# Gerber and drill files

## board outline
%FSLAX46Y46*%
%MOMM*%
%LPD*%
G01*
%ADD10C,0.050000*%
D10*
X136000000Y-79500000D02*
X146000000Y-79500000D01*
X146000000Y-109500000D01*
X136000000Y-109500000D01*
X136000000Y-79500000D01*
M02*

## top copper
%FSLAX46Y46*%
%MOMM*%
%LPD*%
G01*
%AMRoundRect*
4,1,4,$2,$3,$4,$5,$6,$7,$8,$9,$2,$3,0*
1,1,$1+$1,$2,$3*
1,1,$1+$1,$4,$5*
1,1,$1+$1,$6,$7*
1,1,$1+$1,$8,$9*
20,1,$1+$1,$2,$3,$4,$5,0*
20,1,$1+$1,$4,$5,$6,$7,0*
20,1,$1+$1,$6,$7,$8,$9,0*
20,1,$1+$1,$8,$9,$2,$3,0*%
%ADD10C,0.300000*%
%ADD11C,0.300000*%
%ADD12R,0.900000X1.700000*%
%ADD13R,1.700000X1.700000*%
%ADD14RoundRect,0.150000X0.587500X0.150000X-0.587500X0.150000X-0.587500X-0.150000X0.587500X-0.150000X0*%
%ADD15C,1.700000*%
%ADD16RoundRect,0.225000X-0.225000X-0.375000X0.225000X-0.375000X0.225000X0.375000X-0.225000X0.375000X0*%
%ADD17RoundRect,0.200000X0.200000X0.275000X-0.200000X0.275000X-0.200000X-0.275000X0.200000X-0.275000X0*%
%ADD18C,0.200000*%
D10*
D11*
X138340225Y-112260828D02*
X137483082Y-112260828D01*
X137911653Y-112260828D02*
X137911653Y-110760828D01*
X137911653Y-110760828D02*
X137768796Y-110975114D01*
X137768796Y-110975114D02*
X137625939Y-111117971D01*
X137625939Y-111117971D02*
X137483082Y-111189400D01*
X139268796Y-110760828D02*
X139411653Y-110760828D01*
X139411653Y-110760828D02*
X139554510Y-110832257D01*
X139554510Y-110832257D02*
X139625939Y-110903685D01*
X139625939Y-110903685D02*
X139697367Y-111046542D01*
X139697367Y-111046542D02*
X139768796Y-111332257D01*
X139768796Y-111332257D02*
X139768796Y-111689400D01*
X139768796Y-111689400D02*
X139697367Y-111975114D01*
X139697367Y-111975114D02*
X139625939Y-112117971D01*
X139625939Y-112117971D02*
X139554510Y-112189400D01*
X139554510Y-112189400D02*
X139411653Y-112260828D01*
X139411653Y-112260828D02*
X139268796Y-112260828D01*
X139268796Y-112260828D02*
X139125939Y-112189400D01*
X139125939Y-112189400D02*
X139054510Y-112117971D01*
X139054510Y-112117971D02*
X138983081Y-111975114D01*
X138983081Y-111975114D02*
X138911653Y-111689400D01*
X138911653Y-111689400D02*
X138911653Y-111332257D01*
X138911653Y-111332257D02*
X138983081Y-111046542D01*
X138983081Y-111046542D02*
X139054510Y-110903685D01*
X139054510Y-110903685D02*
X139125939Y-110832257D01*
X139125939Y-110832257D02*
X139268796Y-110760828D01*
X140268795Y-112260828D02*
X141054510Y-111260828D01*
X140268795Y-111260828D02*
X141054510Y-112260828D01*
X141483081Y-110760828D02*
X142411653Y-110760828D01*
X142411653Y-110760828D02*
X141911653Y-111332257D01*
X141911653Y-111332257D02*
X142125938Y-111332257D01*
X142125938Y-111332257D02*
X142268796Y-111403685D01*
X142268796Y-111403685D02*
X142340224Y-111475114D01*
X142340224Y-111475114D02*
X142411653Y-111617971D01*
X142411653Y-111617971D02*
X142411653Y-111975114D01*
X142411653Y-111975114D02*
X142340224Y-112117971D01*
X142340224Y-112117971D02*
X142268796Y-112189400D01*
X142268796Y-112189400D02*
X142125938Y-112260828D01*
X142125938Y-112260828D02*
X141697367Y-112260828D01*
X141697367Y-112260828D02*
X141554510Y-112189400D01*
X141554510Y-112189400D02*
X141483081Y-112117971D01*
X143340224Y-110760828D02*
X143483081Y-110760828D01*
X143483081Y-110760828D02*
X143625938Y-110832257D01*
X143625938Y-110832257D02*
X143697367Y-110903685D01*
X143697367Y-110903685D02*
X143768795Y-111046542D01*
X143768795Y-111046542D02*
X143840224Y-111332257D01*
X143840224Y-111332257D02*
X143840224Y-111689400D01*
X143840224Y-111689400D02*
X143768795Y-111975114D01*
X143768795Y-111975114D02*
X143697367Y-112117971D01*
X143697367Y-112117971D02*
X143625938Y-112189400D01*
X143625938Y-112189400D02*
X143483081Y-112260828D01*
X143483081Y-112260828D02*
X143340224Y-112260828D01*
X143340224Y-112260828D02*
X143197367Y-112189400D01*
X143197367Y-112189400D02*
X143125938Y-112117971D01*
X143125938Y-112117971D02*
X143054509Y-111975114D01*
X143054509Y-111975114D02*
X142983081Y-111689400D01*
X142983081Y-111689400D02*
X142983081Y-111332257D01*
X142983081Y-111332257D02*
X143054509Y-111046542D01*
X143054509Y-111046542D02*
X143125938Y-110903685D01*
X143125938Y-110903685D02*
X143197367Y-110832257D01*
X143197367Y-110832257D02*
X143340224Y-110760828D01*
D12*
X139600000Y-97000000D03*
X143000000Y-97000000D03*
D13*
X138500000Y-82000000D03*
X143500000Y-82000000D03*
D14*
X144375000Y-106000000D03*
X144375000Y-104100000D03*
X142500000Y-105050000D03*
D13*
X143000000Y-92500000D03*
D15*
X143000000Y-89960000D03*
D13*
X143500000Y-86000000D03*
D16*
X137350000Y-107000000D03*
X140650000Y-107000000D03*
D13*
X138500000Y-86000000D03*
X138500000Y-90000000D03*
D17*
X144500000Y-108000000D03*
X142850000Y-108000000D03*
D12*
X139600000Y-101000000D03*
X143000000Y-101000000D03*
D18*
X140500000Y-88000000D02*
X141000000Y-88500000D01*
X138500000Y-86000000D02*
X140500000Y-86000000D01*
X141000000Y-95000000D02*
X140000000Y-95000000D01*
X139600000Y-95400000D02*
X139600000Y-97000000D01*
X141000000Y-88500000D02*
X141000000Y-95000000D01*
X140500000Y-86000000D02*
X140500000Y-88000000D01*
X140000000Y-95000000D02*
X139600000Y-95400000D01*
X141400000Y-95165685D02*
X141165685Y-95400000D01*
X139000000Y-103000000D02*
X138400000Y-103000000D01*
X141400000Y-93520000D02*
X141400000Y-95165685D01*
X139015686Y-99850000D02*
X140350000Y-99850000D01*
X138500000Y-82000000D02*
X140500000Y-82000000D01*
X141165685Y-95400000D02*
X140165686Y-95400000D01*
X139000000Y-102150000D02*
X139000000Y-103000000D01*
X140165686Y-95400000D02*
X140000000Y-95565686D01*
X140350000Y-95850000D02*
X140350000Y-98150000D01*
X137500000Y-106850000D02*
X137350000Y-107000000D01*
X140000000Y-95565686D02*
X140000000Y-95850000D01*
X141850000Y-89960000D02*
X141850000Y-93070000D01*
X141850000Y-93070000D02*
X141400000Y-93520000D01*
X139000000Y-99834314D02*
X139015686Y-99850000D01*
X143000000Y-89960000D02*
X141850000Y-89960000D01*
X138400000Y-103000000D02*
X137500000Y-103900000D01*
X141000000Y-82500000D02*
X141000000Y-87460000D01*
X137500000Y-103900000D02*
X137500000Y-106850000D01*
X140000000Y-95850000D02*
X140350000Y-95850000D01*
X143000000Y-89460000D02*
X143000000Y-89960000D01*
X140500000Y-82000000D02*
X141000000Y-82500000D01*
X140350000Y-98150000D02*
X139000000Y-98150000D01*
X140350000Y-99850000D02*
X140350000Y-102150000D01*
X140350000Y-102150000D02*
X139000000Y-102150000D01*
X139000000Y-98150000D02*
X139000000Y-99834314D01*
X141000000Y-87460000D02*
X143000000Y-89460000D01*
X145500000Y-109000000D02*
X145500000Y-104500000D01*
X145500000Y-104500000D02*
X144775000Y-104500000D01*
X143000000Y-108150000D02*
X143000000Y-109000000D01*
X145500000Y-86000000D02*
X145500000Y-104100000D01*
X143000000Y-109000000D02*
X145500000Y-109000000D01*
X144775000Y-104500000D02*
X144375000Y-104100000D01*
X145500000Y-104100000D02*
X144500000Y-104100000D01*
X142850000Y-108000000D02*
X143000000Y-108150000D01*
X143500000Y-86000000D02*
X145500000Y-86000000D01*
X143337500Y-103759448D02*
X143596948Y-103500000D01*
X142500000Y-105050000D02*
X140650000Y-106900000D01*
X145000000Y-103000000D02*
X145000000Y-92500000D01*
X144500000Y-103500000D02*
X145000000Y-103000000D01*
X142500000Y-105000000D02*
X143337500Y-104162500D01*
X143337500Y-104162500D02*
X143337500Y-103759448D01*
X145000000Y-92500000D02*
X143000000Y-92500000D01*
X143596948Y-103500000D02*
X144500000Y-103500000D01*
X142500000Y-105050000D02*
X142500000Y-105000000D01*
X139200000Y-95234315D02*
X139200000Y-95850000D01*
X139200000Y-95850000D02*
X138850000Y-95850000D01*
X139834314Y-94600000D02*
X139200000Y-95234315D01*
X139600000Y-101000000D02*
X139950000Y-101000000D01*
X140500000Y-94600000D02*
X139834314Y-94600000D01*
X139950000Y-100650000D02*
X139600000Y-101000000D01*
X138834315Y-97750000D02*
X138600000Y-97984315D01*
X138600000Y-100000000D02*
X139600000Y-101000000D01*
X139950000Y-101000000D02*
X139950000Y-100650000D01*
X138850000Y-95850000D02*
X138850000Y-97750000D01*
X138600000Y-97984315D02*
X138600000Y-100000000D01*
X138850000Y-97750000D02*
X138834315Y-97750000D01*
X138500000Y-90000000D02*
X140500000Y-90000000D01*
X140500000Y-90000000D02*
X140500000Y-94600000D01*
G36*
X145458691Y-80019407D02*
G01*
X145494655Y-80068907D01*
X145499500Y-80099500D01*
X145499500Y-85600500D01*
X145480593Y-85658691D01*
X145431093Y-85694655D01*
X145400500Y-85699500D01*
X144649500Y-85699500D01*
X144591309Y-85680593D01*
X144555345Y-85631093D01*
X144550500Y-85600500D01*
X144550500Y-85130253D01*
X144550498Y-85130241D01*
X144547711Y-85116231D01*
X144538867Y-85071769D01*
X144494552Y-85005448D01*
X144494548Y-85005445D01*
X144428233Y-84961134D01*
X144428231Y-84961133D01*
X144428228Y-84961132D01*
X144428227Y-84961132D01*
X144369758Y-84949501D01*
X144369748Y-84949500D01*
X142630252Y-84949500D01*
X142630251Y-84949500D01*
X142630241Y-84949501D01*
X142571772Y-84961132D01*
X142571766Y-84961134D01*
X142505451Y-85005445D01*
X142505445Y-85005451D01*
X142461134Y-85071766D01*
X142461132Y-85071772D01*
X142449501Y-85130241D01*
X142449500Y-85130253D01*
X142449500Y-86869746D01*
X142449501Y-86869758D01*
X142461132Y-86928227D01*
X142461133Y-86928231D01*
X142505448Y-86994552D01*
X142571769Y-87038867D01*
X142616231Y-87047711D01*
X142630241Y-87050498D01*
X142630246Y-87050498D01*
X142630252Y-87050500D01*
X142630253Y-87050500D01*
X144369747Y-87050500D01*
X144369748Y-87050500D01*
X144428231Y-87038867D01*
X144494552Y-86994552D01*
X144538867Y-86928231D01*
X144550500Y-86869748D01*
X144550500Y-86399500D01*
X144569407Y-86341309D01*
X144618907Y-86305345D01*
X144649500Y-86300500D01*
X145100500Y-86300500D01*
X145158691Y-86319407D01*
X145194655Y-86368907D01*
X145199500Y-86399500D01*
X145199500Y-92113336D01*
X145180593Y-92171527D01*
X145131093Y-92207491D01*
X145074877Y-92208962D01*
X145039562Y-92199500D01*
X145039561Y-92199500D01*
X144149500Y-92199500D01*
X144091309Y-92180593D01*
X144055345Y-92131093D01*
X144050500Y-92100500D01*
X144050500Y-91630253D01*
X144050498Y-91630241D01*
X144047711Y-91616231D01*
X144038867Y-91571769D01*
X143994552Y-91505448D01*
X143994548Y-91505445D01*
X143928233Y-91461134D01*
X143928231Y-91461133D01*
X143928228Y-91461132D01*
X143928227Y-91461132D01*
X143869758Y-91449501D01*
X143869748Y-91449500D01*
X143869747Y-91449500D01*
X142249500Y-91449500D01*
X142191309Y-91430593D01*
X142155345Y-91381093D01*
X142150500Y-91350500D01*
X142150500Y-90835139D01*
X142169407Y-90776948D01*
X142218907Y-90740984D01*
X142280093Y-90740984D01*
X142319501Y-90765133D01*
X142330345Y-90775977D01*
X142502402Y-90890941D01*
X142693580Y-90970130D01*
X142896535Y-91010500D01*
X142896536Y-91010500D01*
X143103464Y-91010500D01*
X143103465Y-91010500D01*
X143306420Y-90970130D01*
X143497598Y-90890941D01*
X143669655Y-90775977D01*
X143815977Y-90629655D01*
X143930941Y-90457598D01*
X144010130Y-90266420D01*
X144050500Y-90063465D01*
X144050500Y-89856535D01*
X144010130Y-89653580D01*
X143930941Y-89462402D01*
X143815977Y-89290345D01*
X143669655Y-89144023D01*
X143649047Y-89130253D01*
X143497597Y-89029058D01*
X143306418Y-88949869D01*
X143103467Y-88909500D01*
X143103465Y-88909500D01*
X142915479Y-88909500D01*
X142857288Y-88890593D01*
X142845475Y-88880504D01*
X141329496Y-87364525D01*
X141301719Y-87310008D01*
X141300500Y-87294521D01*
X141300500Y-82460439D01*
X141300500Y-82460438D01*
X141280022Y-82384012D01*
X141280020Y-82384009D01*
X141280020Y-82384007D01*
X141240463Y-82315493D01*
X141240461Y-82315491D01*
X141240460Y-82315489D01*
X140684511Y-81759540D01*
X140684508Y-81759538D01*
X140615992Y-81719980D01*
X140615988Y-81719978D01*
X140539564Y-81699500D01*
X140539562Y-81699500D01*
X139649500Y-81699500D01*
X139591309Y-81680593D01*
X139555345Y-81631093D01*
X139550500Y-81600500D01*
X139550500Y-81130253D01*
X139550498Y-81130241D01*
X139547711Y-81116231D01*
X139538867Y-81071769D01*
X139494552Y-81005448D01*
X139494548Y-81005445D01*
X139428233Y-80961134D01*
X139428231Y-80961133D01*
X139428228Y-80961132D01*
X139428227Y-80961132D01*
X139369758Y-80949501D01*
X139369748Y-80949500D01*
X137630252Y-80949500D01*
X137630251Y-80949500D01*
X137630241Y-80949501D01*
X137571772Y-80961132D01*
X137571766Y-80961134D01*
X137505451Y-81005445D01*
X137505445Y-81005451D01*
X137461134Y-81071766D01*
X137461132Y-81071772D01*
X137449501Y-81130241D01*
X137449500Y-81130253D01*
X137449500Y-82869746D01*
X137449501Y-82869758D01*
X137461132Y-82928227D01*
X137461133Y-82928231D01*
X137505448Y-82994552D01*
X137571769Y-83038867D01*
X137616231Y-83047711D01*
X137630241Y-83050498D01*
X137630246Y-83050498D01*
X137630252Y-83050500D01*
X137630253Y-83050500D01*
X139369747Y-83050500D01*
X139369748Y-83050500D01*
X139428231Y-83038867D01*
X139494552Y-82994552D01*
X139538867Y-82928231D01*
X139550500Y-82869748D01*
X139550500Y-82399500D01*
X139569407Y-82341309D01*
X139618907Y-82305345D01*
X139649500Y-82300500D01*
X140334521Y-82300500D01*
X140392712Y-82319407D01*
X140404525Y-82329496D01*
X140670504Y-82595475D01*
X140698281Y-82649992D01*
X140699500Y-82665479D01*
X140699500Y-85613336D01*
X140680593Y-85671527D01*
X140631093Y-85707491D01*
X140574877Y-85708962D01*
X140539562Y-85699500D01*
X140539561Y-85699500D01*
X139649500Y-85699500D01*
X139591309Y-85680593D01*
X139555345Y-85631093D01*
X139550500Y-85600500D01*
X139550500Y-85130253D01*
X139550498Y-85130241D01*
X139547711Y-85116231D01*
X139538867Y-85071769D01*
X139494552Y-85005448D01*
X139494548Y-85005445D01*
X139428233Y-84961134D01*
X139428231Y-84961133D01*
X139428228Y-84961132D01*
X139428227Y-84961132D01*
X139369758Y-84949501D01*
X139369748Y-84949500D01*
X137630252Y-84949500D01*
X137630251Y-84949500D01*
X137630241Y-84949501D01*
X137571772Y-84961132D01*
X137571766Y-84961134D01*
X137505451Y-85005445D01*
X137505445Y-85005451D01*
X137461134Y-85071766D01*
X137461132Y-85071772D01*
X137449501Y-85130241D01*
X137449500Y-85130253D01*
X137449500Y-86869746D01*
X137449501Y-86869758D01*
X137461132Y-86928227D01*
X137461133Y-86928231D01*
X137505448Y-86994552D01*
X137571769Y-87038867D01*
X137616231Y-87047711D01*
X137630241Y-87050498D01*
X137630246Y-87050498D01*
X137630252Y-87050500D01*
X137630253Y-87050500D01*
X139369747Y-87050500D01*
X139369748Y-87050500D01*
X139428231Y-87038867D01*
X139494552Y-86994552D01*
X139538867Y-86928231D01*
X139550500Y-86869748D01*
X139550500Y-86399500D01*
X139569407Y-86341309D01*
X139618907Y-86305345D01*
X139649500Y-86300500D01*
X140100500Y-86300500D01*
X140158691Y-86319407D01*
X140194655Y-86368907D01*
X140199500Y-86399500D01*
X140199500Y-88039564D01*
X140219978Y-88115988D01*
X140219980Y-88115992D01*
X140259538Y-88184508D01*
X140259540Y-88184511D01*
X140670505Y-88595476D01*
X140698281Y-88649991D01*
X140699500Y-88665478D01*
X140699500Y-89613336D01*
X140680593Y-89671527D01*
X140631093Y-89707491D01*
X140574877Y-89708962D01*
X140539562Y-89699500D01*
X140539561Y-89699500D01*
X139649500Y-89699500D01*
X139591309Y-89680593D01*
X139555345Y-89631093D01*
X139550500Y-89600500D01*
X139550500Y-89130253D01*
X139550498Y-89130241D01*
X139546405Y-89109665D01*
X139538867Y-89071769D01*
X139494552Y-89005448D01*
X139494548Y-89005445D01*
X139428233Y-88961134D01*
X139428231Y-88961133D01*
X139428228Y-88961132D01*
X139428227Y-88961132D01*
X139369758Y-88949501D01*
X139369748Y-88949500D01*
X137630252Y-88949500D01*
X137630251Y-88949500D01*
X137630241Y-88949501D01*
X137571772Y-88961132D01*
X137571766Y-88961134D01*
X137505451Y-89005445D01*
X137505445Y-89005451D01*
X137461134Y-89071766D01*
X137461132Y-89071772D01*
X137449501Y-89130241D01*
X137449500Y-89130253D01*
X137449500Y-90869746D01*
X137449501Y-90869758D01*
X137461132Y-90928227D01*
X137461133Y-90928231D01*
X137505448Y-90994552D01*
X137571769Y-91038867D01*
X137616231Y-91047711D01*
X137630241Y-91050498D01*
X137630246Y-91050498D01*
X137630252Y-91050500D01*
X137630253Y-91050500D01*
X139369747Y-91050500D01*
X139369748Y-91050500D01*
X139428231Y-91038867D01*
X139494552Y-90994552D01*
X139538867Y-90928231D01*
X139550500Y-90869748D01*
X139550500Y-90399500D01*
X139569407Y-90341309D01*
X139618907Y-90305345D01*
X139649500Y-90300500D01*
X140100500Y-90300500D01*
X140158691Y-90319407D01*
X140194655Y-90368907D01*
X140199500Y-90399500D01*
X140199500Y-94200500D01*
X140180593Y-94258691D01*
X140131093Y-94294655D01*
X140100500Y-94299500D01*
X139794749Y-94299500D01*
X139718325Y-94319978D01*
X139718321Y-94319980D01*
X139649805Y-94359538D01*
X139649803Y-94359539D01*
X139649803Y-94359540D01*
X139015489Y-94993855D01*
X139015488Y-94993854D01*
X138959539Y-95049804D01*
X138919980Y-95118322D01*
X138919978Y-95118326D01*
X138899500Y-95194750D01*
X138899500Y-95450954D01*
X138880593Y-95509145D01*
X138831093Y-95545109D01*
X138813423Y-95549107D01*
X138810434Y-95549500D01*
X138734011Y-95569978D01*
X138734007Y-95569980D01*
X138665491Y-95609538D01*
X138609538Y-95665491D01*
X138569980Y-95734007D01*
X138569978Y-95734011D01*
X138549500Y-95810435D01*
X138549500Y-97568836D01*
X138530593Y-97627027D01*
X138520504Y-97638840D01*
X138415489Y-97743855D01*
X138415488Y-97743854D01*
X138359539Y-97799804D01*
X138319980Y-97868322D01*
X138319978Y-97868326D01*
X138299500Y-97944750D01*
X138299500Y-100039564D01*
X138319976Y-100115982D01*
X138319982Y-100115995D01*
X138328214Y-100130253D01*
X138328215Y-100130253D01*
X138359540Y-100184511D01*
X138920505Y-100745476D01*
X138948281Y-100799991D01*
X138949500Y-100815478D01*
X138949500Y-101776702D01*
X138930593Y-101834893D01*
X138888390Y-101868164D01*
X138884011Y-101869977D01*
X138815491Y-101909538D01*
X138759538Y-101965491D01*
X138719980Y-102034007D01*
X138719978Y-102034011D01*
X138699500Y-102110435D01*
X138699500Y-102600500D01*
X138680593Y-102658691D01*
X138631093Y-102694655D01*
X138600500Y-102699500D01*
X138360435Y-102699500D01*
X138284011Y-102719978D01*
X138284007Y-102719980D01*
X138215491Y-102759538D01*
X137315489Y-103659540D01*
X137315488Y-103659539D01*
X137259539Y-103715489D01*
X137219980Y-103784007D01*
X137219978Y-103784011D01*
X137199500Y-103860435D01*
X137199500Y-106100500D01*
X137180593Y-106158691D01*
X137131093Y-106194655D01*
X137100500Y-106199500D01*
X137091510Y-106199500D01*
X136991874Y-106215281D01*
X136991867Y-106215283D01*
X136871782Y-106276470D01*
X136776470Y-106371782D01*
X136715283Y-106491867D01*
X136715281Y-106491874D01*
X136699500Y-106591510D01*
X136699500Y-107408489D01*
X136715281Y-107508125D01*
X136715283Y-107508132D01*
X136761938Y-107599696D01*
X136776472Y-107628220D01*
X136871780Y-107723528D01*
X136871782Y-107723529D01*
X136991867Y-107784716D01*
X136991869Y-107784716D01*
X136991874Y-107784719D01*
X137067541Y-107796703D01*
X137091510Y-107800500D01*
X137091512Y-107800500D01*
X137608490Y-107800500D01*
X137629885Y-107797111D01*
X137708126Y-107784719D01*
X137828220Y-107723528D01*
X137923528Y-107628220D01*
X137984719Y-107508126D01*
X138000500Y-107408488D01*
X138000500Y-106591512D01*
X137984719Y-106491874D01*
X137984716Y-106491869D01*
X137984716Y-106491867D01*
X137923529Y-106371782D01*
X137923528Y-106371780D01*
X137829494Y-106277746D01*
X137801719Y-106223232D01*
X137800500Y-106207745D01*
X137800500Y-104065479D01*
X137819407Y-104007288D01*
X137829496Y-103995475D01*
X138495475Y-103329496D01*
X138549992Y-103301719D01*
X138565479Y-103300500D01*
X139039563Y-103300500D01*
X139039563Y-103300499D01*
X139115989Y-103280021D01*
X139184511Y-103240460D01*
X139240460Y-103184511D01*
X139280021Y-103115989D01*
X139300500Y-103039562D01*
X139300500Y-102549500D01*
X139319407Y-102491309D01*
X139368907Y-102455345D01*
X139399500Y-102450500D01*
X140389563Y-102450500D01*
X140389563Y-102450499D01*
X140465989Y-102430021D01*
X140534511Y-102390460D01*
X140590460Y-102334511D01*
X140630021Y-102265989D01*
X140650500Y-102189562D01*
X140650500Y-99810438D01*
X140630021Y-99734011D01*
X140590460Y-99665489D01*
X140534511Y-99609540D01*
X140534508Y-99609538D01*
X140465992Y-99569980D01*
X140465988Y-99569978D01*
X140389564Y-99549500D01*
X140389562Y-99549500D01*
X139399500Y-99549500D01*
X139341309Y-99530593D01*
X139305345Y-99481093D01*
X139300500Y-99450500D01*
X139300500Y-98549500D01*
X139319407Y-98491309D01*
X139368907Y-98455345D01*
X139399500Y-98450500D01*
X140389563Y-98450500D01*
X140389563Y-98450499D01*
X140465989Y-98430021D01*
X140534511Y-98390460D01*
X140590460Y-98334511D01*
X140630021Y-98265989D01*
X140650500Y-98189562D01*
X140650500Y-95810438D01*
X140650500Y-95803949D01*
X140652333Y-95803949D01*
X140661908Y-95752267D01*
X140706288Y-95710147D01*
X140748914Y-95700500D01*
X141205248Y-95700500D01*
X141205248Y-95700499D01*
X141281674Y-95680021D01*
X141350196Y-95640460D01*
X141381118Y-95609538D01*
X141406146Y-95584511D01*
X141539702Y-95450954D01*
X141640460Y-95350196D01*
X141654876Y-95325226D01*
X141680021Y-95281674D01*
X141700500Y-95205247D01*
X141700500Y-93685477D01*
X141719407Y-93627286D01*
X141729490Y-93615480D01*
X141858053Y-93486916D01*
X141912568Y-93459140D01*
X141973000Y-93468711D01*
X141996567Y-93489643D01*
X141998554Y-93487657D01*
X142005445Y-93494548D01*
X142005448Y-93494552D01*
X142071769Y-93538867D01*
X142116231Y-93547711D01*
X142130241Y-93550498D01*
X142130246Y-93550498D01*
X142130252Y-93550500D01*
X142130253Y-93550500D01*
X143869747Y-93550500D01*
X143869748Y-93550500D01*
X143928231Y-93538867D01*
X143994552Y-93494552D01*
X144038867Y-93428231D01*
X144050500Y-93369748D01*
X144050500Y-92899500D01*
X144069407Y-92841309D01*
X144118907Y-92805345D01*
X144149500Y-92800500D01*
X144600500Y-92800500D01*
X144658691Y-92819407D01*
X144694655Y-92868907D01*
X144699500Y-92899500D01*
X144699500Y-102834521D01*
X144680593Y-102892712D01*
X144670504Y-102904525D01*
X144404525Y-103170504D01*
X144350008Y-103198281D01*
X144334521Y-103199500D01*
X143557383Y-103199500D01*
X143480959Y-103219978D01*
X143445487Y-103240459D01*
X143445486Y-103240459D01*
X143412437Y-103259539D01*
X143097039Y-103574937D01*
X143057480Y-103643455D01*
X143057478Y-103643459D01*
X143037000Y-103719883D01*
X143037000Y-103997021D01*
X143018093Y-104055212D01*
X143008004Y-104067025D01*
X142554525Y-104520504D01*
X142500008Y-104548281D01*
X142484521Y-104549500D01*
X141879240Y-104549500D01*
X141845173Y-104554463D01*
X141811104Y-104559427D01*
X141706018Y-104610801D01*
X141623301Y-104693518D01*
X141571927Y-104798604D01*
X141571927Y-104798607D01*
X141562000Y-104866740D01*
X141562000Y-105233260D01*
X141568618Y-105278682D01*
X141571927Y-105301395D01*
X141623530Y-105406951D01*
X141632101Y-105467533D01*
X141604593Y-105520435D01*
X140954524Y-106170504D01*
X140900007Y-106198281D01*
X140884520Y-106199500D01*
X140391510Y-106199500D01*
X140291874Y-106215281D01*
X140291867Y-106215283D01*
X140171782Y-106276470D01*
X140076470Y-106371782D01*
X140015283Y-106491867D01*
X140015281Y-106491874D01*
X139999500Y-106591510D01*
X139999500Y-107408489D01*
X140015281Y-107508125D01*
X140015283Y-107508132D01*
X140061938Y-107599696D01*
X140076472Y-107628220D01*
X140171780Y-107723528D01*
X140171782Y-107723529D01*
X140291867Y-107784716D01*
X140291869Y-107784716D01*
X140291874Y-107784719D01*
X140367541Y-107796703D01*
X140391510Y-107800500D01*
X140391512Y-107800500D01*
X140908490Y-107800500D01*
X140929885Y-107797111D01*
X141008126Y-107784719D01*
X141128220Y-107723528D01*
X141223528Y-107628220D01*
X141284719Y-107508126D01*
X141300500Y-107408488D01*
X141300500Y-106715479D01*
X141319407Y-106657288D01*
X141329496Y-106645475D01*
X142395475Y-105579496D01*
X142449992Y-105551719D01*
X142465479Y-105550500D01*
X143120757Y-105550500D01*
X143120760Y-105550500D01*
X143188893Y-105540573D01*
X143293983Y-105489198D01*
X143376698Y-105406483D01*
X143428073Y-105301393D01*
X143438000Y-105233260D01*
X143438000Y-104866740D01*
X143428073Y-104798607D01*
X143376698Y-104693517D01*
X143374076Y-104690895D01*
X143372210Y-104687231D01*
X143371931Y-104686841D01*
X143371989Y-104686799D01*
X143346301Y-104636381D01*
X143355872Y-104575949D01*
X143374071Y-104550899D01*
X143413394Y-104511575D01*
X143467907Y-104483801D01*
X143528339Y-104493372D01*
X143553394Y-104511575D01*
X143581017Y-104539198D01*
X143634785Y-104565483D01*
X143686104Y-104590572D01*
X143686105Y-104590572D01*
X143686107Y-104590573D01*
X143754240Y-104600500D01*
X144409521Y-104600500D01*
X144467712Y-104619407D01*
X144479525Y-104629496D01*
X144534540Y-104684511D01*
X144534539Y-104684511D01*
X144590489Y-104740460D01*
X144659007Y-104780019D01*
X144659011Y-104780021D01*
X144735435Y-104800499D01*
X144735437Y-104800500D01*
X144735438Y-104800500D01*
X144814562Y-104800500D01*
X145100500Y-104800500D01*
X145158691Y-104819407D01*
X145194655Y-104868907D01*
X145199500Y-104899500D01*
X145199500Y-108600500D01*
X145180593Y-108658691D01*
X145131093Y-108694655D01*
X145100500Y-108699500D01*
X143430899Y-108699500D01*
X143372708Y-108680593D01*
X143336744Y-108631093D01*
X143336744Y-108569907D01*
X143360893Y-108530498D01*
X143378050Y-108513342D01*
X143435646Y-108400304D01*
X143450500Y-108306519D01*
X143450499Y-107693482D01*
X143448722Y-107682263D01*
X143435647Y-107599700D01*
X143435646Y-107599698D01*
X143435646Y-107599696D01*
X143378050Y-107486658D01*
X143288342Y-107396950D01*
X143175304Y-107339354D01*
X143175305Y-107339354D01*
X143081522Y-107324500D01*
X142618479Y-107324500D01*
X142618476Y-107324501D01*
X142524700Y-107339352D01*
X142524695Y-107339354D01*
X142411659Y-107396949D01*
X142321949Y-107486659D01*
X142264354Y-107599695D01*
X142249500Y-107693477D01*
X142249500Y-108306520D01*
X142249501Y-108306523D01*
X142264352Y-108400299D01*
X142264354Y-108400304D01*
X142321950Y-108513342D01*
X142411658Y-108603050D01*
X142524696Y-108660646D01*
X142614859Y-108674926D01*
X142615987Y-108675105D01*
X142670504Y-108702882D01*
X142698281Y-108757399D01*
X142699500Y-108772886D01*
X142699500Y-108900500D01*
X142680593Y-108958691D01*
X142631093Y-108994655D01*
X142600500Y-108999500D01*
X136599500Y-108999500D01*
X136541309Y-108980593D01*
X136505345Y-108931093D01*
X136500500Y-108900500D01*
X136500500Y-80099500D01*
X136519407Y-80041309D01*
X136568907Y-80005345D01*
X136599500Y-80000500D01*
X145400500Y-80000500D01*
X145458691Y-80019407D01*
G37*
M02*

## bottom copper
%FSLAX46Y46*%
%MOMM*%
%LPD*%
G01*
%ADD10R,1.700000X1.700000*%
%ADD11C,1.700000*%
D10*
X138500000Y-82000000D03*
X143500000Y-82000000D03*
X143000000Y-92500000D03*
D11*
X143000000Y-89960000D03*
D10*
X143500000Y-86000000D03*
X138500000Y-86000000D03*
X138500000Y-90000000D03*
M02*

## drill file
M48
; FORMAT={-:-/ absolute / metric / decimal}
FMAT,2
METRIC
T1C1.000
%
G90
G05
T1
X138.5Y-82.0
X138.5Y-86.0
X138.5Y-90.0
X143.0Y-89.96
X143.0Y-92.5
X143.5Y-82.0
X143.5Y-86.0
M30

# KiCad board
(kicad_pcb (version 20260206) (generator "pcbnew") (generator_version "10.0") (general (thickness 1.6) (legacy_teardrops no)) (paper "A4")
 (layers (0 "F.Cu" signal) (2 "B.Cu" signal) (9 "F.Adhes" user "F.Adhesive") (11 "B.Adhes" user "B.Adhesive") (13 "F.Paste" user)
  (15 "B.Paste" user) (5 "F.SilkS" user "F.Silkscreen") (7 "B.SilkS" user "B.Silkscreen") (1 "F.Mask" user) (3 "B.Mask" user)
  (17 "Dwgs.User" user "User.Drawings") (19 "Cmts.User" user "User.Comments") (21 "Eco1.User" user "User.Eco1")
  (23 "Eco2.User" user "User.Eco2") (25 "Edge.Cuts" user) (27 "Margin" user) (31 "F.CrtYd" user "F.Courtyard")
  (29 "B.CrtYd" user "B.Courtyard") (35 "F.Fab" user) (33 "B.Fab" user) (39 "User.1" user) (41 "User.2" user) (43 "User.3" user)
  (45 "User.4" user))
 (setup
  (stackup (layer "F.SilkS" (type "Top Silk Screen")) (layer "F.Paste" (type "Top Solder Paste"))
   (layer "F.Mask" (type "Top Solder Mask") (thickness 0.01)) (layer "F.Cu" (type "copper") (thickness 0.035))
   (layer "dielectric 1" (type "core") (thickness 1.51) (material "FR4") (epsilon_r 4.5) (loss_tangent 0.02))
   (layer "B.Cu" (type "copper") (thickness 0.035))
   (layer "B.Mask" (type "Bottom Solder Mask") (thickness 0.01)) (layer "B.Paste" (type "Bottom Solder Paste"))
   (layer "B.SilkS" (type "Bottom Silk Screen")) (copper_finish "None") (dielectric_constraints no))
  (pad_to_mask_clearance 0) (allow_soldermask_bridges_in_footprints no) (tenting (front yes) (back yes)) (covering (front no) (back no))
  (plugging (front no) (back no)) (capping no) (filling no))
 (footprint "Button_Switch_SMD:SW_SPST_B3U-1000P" (layer "F.Cu") (at 141.3 97)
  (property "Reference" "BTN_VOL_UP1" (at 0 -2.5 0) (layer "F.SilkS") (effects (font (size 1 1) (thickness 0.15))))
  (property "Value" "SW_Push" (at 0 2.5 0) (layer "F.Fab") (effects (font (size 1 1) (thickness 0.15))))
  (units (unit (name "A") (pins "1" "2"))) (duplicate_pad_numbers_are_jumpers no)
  (pad "1" smd rect (at -1.7 0) (size 0.9 1.7) (layers "F.Cu" "F.Mask" "F.Paste") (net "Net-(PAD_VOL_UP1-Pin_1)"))
  (pad "2" smd rect (at 1.7 0) (size 0.9 1.7) (layers "F.Cu" "F.Mask" "F.Paste") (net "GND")))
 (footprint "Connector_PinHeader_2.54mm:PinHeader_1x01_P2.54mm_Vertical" (layer "F.Cu") (at 138.5 82)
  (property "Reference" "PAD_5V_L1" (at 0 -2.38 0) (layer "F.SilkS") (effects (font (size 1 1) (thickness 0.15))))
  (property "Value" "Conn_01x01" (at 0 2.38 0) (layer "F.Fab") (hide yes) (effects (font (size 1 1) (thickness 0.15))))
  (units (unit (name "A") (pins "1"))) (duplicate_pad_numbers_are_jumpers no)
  (pad "1" thru_hole rect (at 0 0) (size 1.7 1.7) (drill 1) (layers "*.Cu" "*.Mask") (remove_unused_layers no) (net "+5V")))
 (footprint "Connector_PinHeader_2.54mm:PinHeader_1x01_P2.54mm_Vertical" (layer "F.Cu") (at 143.5 82)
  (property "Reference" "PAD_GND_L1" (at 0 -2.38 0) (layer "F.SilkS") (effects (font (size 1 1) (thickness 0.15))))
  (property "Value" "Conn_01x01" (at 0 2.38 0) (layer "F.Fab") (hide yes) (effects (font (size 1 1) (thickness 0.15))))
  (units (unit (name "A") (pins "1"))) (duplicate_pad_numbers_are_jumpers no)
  (pad "1" thru_hole rect (at 0 0) (size 1.7 1.7) (drill 1) (layers "*.Cu" "*.Mask") (remove_unused_layers no) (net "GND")))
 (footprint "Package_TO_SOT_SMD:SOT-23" (layer "F.Cu") (at 143.4375 105.05 180)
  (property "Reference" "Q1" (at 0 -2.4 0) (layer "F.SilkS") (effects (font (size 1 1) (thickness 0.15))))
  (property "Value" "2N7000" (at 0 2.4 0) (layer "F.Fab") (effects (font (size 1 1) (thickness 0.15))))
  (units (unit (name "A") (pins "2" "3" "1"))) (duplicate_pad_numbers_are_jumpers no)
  (pad "1" smd roundrect (at -0.9375 -0.95 180) (size 1.475 0.6) (layers "F.Cu" "F.Mask" "F.Paste") (roundrect_rratio 0.25) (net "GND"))
  (pad "2" smd roundrect (at -0.9375 0.95 180) (size 1.475 0.6) (layers "F.Cu" "F.Mask" "F.Paste") (roundrect_rratio 0.25)
   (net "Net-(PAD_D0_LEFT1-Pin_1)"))
  (pad "3" smd roundrect (at 0.9375 0 180) (size 1.475 0.6) (layers "F.Cu" "F.Mask" "F.Paste") (roundrect_rratio 0.25) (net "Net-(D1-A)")))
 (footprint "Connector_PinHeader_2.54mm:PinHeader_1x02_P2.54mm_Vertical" (layer "F.Cu") (at 143 92.5 180)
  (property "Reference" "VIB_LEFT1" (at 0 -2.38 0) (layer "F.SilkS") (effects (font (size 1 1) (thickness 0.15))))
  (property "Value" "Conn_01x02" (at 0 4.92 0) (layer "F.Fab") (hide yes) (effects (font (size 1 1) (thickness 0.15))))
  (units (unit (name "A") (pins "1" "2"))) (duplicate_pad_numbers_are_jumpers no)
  (pad "1" thru_hole rect (at 0 0 180) (size 1.7 1.7) (drill 1) (layers "*.Cu" "*.Mask") (remove_unused_layers no) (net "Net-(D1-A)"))
  (pad "2" thru_hole circle (at 0 2.54 180) (size 1.7 1.7) (drill 1) (layers "*.Cu" "*.Mask") (remove_unused_layers no) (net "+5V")))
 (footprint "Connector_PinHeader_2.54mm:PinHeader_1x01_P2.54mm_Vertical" (layer "F.Cu") (at 143.5 86)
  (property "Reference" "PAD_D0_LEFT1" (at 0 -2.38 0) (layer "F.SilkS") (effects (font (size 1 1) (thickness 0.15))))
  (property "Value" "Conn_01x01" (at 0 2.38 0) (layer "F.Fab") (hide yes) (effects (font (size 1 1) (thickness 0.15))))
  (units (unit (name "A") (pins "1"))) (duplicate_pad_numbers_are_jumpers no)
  (pad "1" thru_hole rect (at 0 0) (size 1.7 1.7) (drill 1) (layers "*.Cu" "*.Mask") (remove_unused_layers no)
   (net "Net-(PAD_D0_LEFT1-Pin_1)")))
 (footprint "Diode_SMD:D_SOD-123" (layer "F.Cu") (at 139 107)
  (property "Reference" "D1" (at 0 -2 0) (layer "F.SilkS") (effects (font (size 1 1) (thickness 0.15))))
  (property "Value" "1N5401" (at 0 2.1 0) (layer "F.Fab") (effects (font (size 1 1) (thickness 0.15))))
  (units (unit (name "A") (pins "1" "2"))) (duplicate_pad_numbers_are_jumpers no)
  (pad "1" smd roundrect (at -1.65 0) (size 0.9 1.2) (layers "F.Cu" "F.Mask" "F.Paste") (roundrect_rratio 0.25) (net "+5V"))
  (pad "2" smd roundrect (at 1.65 0) (size 0.9 1.2) (layers "F.Cu" "F.Mask" "F.Paste") (roundrect_rratio 0.25) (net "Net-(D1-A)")))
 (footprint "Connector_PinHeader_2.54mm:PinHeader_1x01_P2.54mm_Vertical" (layer "F.Cu") (at 138.5 86)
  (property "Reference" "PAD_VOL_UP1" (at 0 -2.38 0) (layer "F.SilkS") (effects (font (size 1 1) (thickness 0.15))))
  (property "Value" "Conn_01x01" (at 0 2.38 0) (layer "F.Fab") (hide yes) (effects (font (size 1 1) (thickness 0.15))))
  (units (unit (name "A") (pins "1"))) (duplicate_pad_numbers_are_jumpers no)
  (pad "1" thru_hole rect (at 0 0) (size 1.7 1.7) (drill 1) (layers "*.Cu" "*.Mask") (remove_unused_layers no)
   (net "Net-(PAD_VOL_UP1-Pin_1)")))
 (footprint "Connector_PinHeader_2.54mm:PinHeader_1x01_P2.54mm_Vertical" (layer "F.Cu") (at 138.5 90)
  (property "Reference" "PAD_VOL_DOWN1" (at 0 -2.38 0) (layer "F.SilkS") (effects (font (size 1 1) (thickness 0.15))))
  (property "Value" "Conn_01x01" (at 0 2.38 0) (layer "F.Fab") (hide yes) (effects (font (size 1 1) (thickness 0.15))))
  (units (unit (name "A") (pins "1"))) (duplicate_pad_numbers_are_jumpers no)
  (pad "1" thru_hole rect (at 0 0) (size 1.7 1.7) (drill 1) (layers "*.Cu" "*.Mask") (remove_unused_layers no)
   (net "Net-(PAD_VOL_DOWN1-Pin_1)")))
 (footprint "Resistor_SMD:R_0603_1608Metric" (layer "F.Cu") (at 143.675 108 180)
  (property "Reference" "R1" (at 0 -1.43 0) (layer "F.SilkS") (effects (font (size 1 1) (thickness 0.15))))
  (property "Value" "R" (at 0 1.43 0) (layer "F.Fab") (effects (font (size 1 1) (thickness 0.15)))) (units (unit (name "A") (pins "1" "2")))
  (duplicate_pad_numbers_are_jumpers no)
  (pad "1" smd roundrect (at -0.825 0 180) (size 0.8 0.95) (layers "F.Cu" "F.Mask" "F.Paste") (roundrect_rratio 0.25) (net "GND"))
  (pad "2" smd roundrect (at 0.825 0 180) (size 0.8 0.95) (layers "F.Cu" "F.Mask" "F.Paste") (roundrect_rratio 0.25)
   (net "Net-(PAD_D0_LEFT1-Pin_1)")))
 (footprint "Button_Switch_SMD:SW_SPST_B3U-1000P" (layer "F.Cu") (at 141.3 101)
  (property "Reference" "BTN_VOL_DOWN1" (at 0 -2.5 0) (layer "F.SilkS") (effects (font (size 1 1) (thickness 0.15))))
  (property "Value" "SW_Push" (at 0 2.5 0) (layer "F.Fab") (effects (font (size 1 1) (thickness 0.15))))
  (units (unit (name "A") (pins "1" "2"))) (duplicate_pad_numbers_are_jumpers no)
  (pad "1" smd rect (at -1.7 0) (size 0.9 1.7) (layers "F.Cu" "F.Mask" "F.Paste") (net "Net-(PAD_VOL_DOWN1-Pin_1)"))
  (pad "2" smd rect (at 1.7 0) (size 0.9 1.7) (layers "F.Cu" "F.Mask" "F.Paste") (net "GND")))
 (gr_rect (start 136 79.5) (end 146 109.5) (stroke (width 0.05) (type default)) (fill no) (layer "Edge.Cuts"))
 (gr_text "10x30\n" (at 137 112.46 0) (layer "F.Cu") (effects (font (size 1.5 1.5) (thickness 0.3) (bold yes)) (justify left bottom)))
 (segment (start 140.5 88) (end 141 88.5) (width 0.2) (layer "F.Cu") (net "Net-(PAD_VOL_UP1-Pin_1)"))
 (segment (start 138.5 86) (end 140.5 86) (width 0.2) (layer "F.Cu") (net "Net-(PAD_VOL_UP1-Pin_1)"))
 (segment (start 141 95) (end 140 95) (width 0.2) (layer "F.Cu") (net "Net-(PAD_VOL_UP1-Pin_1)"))
 (segment (start 139.6 95.4) (end 139.6 97) (width 0.2) (layer "F.Cu") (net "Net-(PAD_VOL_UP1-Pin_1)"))
 (segment (start 141 88.5) (end 141 95) (width 0.2) (layer "F.Cu") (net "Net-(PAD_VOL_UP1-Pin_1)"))
 (segment (start 140.5 86) (end 140.5 88) (width 0.2) (layer "F.Cu") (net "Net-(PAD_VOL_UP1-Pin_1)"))
 (segment (start 140 95) (end 139.6 95.4) (width 0.2) (layer "F.Cu") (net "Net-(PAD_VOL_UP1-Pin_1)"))
 (segment (start 141.4 95.165685) (end 141.165685 95.4) (width 0.2) (layer "F.Cu") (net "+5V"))
 (segment (start 139 103) (end 138.4 103) (width 0.2) (layer "F.Cu") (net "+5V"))
 (segment (start 141.4 93.52) (end 141.4 95.165685) (width 0.2) (layer "F.Cu") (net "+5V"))
 (segment (start 139.015686 99.85) (end 140.35 99.85) (width 0.2) (layer "F.Cu") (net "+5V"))
 (segment (start 138.5 82) (end 140.5 82) (width 0.2) (layer "F.Cu") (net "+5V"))
 (segment (start 141.165685 95.4) (end 140.165686 95.4) (width 0.2) (layer "F.Cu") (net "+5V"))
 (segment (start 139 102.15) (end 139 103) (width 0.2) (layer "F.Cu") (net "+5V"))
 (segment (start 140.165686 95.4) (end 140 95.565686) (width 0.2) (layer "F.Cu") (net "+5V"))
 (segment (start 140.35 95.85) (end 140.35 98.15) (width 0.2) (layer "F.Cu") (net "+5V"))
 (segment (start 137.5 106.85) (end 137.35 107) (width 0.2) (layer "F.Cu") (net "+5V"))
 (segment (start 140 95.565686) (end 140 95.85) (width 0.2) (layer "F.Cu") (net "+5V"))
 (segment (start 141.85 89.96) (end 141.85 93.07) (width 0.2) (layer "F.Cu") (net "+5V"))
 (segment (start 141.85 93.07) (end 141.4 93.52) (width 0.2) (layer "F.Cu") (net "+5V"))
 (segment (start 139 99.834314) (end 139.015686 99.85) (width 0.2) (layer "F.Cu") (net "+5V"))
 (segment (start 143 89.96) (end 141.85 89.96) (width 0.2) (layer "F.Cu") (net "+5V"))
 (segment (start 138.4 103) (end 137.5 103.9) (width 0.2) (layer "F.Cu") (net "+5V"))
 (segment (start 141 82.5) (end 141 87.46) (width 0.2) (layer "F.Cu") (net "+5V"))
 (segment (start 137.5 103.9) (end 137.5 106.85) (width 0.2) (layer "F.Cu") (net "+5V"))
 (segment (start 140 95.85) (end 140.35 95.85) (width 0.2) (layer "F.Cu") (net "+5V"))
 (segment (start 143 89.46) (end 143 89.96) (width 0.2) (layer "F.Cu") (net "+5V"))
 (segment (start 140.5 82) (end 141 82.5) (width 0.2) (layer "F.Cu") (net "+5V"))
 (segment (start 140.35 98.15) (end 139 98.15) (width 0.2) (layer "F.Cu") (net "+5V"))
 (segment (start 140.35 99.85) (end 140.35 102.15) (width 0.2) (layer "F.Cu") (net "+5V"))
 (segment (start 140.35 102.15) (end 139 102.15) (width 0.2) (layer "F.Cu") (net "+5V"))
 (segment (start 139 98.15) (end 139 99.834314) (width 0.2) (layer "F.Cu") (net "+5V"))
 (segment (start 141 87.46) (end 143 89.46) (width 0.2) (layer "F.Cu") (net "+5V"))
 (segment (start 145.5 109) (end 145.5 104.5) (width 0.2) (layer "F.Cu") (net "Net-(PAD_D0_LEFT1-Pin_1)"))
 (segment (start 145.5 104.5) (end 144.775 104.5) (width 0.2) (layer "F.Cu") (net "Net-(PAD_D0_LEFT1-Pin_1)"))
 (segment (start 143 108.15) (end 143 109) (width 0.2) (layer "F.Cu") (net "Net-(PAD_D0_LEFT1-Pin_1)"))
 (segment (start 145.5 86) (end 145.5 104.1) (width 0.2) (layer "F.Cu") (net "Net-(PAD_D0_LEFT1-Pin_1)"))
 (segment (start 143 109) (end 145.5 109) (width 0.2) (layer "F.Cu") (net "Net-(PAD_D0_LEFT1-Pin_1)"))
 (segment (start 144.775 104.5) (end 144.375 104.1) (width 0.2) (layer "F.Cu") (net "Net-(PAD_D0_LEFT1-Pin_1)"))
 (segment (start 145.5 104.1) (end 144.5 104.1) (width 0.2) (layer "F.Cu") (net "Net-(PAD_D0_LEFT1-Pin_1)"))
 (segment (start 142.85 108) (end 143 108.15) (width 0.2) (layer "F.Cu") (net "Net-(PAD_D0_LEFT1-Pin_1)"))
 (segment (start 143.5 86) (end 145.5 86) (width 0.2) (layer "F.Cu") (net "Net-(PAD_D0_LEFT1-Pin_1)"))
 (segment (start 143.3375 103.759448) (end 143.596948 103.5) (width 0.2) (layer "F.Cu") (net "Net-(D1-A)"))
 (segment (start 142.5 105.05) (end 140.65 106.9) (width 0.2) (layer "F.Cu") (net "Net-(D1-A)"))
 (segment (start 145 103) (end 145 92.5) (width 0.2) (layer "F.Cu") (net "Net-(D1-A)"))
 (segment (start 144.5 103.5) (end 145 103) (width 0.2) (layer "F.Cu") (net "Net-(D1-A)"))
 (segment (start 142.5 105) (end 143.3375 104.1625) (width 0.2) (layer "F.Cu") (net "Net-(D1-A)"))
 (segment (start 143.3375 104.1625) (end 143.3375 103.759448) (width 0.2) (layer "F.Cu") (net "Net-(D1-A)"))
 (segment (start 145 92.5) (end 143 92.5) (width 0.2) (layer "F.Cu") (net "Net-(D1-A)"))
 (segment (start 143.596948 103.5) (end 144.5 103.5) (width 0.2) (layer "F.Cu") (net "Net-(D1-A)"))
 (segment (start 142.5 105.05) (end 142.5 105) (width 0.2) (layer "F.Cu") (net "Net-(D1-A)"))
 (segment (start 139.2 95.234315) (end 139.2 95.85) (width 0.2) (layer "F.Cu") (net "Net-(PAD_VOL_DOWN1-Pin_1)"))
 (segment (start 139.2 95.85) (end 138.85 95.85) (width 0.2) (layer "F.Cu") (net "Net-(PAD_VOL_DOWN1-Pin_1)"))
 (segment (start 139.834314 94.6) (end 139.2 95.234315) (width 0.2) (layer "F.Cu") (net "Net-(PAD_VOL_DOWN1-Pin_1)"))
 (segment (start 139.6 101) (end 139.95 101) (width 0.2) (layer "F.Cu") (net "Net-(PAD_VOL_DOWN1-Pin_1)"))
 (segment (start 140.5 94.6) (end 139.834314 94.6) (width 0.2) (layer "F.Cu") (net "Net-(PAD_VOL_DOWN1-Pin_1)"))
 (segment (start 139.95 100.65) (end 139.6 101) (width 0.2) (layer "F.Cu") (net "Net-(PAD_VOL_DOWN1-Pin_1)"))
 (segment (start 138.834315 97.75) (end 138.6 97.984315) (width 0.2) (layer "F.Cu") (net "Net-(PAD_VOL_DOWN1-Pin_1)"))
 (segment (start 138.6 100) (end 139.6 101) (width 0.2) (layer "F.Cu") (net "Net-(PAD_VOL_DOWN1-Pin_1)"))
 (segment (start 139.95 101) (end 139.95 100.65) (width 0.2) (layer "F.Cu") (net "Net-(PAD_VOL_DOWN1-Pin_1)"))
 (segment (start 138.85 95.85) (end 138.85 97.75) (width 0.2) (layer "F.Cu") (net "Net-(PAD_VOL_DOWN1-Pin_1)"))
 (segment (start 138.6 97.984315) (end 138.6 100) (width 0.2) (layer "F.Cu") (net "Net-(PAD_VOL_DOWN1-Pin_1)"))
 (segment (start 138.85 97.75) (end 138.834315 97.75) (width 0.2) (layer "F.Cu") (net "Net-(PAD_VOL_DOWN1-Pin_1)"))
 (segment (start 138.5 90) (end 140.5 90) (width 0.2) (layer "F.Cu") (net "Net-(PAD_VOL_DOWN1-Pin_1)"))
 (segment (start 140.5 90) (end 140.5 94.6) (width 0.2) (layer "F.Cu") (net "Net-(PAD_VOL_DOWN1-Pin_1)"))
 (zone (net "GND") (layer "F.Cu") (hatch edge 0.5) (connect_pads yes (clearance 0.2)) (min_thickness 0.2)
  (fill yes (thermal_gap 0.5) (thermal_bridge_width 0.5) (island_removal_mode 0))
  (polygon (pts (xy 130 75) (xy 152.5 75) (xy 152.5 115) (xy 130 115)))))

